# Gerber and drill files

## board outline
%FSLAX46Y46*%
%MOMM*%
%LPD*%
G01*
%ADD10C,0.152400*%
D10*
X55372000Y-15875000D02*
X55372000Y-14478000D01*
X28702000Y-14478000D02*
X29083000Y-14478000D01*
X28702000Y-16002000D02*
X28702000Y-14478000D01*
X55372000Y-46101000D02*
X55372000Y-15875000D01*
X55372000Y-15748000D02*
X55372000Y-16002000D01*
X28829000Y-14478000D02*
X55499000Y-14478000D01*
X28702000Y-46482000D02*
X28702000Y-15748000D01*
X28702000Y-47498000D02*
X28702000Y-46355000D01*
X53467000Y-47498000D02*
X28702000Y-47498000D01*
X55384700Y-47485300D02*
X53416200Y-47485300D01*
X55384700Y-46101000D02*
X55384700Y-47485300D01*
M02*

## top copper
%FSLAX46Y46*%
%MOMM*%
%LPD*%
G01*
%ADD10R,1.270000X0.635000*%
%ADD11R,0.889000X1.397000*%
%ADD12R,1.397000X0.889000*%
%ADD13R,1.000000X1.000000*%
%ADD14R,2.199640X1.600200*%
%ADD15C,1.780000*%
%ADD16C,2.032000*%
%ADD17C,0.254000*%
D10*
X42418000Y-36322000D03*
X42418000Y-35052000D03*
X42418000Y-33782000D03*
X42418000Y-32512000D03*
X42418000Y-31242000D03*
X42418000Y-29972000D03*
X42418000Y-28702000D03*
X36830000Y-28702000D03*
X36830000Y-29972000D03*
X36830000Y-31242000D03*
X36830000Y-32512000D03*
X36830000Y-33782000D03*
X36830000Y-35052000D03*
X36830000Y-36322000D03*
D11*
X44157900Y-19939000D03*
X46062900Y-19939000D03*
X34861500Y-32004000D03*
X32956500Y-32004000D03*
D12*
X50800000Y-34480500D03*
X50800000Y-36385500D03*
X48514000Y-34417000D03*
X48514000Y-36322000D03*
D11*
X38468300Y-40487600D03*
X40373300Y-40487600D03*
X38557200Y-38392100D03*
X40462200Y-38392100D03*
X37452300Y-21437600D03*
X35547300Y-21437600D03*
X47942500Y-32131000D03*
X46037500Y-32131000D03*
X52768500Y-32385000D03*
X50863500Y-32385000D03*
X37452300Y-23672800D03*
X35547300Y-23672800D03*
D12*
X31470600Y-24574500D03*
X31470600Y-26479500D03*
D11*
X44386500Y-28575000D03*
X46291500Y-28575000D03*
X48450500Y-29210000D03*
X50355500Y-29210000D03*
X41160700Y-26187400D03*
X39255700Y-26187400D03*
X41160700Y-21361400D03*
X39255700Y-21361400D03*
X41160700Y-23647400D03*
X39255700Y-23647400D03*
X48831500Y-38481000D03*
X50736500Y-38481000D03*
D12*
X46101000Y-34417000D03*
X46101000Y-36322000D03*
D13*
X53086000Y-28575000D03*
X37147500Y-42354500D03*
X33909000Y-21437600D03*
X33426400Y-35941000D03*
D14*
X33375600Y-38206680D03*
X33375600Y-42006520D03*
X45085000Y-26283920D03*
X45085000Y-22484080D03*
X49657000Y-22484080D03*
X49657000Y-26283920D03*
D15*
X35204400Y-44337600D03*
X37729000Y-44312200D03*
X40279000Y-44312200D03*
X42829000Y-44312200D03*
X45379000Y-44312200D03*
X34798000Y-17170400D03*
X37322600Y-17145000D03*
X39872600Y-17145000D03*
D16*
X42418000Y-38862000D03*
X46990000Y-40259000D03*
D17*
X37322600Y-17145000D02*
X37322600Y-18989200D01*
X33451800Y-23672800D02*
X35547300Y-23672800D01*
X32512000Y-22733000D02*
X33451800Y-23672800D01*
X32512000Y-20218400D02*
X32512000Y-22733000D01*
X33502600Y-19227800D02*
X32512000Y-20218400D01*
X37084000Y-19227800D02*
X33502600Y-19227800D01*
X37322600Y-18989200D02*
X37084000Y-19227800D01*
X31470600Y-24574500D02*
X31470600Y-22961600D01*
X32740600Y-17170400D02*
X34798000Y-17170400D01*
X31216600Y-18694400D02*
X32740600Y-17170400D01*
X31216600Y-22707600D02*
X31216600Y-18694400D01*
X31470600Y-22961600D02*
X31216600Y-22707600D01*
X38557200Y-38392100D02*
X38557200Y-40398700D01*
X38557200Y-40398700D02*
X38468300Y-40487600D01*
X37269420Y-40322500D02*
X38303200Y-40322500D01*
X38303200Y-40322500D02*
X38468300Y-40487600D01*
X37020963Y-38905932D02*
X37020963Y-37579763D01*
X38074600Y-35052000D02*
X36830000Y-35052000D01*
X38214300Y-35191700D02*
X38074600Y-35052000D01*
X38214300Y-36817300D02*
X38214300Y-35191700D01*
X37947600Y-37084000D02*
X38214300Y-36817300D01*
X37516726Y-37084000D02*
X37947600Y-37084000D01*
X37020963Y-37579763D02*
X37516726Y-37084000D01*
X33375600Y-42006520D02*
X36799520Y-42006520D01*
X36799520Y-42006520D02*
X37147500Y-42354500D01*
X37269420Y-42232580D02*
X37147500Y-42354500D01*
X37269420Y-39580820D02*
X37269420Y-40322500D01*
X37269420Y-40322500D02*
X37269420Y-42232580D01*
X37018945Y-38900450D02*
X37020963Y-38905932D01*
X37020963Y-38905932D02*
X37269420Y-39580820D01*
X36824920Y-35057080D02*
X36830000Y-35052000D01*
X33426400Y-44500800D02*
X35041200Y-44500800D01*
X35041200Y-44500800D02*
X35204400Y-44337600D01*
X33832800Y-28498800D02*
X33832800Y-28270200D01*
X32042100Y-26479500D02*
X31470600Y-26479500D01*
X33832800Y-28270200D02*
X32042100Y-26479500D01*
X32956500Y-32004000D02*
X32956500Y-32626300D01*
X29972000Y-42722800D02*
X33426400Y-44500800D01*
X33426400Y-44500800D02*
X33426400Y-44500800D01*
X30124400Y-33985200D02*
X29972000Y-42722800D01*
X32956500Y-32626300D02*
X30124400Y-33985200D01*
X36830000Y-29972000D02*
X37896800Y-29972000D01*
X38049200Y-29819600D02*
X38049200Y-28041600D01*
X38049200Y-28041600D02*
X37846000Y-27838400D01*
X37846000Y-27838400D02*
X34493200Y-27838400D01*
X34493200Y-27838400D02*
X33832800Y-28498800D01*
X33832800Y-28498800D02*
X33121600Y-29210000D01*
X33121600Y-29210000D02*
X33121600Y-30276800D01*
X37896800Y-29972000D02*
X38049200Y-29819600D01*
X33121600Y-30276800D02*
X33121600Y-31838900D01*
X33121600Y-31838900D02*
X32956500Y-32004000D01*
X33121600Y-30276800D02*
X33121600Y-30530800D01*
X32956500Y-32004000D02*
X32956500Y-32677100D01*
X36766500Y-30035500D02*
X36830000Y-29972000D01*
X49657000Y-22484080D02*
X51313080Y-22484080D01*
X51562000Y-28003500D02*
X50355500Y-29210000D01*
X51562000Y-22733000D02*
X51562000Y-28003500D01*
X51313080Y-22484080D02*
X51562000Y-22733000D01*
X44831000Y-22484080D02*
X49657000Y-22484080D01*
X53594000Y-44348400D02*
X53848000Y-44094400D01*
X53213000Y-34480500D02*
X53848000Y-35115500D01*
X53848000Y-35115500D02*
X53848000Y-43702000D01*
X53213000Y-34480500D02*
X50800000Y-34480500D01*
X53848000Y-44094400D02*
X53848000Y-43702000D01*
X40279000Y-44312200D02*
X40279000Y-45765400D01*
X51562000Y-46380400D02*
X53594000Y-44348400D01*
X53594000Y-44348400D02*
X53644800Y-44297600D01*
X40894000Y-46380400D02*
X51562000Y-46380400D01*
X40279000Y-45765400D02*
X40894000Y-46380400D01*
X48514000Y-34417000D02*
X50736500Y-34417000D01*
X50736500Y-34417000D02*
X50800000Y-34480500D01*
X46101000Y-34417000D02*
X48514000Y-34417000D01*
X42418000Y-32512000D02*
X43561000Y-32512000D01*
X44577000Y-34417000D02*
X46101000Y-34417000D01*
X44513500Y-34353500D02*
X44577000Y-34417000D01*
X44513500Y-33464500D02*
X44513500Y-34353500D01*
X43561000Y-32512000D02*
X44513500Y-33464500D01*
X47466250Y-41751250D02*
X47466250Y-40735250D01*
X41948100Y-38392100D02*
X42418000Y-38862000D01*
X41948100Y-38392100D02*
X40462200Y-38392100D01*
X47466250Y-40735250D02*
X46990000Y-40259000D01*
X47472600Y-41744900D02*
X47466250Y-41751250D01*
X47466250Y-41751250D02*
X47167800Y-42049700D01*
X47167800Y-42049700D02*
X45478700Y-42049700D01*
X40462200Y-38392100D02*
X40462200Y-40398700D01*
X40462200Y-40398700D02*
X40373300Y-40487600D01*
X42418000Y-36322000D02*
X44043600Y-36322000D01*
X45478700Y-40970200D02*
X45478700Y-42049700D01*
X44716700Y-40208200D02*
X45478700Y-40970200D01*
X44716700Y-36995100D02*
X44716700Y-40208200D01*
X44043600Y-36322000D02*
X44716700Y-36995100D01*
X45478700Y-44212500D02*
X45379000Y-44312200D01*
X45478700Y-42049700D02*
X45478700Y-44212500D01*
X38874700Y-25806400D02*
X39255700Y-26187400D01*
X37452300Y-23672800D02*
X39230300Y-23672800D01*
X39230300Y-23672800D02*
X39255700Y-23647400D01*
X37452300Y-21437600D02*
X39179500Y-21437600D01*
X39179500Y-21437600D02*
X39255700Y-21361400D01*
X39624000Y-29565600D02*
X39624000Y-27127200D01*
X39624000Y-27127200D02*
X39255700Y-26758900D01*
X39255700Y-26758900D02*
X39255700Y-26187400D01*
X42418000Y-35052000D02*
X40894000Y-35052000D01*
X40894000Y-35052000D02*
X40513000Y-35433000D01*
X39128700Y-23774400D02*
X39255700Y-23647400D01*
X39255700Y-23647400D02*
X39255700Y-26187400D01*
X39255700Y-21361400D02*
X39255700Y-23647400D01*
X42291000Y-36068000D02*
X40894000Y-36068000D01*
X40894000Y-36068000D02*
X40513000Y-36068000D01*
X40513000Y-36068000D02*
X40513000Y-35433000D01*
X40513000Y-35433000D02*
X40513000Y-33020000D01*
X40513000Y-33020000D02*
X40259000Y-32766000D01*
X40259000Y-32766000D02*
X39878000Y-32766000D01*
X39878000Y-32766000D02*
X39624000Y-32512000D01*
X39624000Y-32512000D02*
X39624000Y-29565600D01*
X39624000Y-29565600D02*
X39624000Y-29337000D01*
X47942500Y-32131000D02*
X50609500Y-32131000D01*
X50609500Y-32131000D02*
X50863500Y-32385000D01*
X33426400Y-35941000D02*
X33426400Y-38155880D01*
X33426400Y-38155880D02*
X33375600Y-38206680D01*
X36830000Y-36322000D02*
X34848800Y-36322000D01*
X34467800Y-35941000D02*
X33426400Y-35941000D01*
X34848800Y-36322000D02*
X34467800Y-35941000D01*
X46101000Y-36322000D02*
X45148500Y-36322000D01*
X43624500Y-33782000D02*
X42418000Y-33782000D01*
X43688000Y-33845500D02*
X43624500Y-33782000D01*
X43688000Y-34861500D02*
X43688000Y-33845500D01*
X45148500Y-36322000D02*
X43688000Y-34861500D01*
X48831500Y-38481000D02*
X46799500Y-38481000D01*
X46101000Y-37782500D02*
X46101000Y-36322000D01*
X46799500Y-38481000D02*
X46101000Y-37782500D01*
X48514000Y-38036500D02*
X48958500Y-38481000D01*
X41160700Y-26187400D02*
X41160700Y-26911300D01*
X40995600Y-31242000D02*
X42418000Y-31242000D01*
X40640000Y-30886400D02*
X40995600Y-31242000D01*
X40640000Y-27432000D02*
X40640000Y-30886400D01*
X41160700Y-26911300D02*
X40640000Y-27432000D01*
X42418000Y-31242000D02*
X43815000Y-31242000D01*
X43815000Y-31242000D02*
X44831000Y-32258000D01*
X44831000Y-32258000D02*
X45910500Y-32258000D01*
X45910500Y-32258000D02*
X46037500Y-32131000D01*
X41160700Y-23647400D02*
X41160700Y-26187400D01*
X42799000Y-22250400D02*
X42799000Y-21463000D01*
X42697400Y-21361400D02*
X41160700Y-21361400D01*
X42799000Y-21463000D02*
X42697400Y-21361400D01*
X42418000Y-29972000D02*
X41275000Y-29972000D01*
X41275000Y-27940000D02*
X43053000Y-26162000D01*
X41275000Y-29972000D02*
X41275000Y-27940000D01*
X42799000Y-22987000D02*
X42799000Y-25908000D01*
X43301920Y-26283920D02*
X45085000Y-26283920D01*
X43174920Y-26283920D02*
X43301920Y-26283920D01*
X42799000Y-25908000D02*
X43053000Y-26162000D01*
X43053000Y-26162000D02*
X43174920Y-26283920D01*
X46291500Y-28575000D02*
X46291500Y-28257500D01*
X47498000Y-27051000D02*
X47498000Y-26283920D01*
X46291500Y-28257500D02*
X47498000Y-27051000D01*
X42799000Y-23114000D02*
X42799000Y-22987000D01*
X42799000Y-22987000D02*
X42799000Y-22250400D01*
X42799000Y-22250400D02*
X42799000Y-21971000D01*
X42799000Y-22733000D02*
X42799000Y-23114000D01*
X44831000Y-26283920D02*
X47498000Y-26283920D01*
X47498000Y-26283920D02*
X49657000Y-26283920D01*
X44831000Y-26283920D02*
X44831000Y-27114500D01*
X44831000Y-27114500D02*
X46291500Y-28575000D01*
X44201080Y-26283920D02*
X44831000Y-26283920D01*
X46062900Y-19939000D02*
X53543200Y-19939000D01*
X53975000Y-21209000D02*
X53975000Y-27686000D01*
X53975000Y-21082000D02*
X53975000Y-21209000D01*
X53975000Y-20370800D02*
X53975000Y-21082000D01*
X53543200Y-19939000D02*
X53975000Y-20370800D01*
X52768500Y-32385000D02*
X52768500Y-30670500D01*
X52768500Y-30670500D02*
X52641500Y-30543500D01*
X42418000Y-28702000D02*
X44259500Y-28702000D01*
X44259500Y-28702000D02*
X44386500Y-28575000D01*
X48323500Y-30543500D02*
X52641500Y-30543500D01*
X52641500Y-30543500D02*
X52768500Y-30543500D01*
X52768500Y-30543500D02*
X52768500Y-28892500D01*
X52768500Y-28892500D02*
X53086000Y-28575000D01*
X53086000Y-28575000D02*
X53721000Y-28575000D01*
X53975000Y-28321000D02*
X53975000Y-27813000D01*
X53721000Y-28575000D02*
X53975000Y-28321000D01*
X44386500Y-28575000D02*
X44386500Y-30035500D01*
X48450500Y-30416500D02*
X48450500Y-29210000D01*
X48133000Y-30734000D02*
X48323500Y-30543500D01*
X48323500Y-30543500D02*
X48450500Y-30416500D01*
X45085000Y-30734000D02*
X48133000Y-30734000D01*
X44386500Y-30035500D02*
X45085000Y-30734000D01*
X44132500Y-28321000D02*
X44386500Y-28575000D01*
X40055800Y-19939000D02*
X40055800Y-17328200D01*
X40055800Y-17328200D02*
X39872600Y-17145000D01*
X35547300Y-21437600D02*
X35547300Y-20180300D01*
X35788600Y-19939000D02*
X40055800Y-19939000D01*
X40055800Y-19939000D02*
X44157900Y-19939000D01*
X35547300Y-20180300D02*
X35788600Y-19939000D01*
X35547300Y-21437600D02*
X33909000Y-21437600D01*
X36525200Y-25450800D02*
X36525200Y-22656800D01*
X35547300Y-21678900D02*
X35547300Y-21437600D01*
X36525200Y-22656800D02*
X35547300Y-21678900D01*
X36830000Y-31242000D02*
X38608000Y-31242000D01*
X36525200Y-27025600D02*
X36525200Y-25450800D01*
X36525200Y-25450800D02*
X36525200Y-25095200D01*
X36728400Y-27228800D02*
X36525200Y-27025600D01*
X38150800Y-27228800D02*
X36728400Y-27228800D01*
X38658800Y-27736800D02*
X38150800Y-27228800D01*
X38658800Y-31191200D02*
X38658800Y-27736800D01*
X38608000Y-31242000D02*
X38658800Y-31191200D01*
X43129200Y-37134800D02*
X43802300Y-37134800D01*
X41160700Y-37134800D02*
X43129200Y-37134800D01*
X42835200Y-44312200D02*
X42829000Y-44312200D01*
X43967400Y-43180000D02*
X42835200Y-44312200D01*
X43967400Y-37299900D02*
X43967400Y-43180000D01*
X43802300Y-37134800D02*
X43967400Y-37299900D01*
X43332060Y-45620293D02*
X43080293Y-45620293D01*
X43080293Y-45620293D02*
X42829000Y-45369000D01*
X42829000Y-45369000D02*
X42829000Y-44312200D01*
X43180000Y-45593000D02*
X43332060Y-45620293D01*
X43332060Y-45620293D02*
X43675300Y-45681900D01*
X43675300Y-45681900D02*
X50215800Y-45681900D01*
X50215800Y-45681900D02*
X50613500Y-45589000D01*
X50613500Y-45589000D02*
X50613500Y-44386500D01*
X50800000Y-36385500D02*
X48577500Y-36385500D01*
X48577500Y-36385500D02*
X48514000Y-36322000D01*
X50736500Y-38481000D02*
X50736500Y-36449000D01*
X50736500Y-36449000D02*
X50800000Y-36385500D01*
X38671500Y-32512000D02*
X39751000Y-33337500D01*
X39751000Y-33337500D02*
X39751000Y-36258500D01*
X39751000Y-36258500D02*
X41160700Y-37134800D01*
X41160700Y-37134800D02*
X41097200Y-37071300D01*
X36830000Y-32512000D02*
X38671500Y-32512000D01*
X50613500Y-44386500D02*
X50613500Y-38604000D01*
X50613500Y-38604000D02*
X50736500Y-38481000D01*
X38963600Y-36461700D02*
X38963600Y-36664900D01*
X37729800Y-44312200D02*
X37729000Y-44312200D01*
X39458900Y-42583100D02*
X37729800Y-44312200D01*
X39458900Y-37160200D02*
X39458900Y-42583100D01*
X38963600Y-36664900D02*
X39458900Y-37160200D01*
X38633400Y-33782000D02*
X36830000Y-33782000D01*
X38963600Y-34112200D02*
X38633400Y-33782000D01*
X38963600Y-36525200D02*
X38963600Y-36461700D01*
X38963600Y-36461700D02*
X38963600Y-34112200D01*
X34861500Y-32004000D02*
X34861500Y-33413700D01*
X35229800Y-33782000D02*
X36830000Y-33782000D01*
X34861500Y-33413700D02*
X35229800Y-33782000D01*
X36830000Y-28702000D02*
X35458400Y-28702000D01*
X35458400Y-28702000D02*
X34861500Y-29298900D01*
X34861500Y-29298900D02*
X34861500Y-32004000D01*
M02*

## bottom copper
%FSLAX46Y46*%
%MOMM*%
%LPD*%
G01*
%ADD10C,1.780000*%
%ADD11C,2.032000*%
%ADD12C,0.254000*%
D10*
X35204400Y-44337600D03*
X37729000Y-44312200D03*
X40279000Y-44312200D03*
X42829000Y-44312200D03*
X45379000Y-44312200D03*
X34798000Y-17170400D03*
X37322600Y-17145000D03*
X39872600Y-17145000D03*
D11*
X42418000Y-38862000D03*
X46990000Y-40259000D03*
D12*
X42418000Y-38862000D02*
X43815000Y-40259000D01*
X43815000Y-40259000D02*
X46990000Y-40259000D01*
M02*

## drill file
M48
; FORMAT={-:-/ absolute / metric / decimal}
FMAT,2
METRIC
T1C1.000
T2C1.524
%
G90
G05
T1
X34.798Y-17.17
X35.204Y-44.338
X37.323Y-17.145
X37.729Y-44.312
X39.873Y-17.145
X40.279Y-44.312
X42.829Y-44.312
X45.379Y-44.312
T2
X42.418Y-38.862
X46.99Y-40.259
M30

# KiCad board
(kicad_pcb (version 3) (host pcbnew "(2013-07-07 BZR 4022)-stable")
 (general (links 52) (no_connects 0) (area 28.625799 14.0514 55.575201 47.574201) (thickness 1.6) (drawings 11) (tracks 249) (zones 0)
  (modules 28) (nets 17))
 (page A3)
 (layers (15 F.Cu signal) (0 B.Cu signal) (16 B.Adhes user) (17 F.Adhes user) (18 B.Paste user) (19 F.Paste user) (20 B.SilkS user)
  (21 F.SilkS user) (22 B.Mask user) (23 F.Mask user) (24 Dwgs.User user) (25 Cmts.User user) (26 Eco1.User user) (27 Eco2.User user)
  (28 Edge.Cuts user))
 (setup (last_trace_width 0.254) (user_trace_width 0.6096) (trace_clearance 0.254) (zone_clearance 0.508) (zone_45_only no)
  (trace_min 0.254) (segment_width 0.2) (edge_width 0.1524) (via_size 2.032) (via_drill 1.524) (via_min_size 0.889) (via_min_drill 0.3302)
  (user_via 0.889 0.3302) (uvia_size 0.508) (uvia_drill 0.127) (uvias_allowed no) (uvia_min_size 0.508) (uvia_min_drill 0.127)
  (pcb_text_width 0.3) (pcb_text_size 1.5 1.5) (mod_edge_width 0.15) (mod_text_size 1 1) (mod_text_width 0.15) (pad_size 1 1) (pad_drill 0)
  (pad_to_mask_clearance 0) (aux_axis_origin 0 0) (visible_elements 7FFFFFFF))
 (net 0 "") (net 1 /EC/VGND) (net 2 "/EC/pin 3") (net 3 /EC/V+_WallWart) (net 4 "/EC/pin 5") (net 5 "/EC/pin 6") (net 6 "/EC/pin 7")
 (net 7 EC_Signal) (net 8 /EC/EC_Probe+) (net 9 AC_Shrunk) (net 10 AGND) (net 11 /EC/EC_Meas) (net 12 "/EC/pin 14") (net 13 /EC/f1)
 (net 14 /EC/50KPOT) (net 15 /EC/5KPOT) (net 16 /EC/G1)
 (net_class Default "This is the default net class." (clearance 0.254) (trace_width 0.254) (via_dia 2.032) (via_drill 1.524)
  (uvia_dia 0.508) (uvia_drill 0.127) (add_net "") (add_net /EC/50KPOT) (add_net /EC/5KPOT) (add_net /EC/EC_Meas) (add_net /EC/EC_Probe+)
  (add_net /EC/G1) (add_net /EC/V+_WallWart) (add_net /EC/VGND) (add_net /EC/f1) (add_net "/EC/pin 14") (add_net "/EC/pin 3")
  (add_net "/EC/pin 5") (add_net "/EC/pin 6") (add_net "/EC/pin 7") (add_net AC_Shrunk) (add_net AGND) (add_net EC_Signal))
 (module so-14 (layer F.Cu) (at 39.624 32.512 90)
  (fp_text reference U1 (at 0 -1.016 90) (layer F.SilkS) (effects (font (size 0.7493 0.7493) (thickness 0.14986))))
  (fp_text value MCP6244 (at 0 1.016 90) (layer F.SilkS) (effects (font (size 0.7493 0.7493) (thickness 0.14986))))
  (pad 1 smd rect (at -3.81 2.794 90) (size 0.635 1.27) (layers F.Cu F.Paste F.Mask) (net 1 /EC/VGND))
  (pad 2 smd rect (at -2.54 2.794 90) (size 0.635 1.27) (layers F.Cu F.Paste F.Mask) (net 1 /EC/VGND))
  (pad 3 smd rect (at -1.27 2.794 90) (size 0.635 1.27) (layers F.Cu F.Paste F.Mask) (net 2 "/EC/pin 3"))
  (pad 4 smd rect (at 0 2.794 90) (size 0.635 1.27) (layers F.Cu F.Paste F.Mask) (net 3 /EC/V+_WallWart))
  (pad 5 smd rect (at 1.27 2.794 90) (size 0.635 1.27) (layers F.Cu F.Paste F.Mask) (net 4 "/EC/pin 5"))
  (pad 6 smd rect (at 2.54 2.794 90) (size 0.635 1.27) (layers F.Cu F.Paste F.Mask) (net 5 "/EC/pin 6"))
  (pad 7 smd rect (at 3.81 2.794 90) (size 0.635 1.27) (layers F.Cu F.Paste F.Mask) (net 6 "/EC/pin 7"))
  (pad 8 smd rect (at 3.81 -2.794 90) (size 0.635 1.27) (layers F.Cu F.Paste F.Mask) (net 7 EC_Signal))
  (pad 9 smd rect (at 2.54 -2.794 90) (size 0.635 1.27) (layers F.Cu F.Paste F.Mask) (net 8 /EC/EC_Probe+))
  (pad 10 smd rect (at 1.27 -2.794 90) (size 0.635 1.27) (layers F.Cu F.Paste F.Mask) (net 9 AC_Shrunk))
  (pad 11 smd rect (at 0 -2.794 90) (size 0.635 1.27) (layers F.Cu F.Paste F.Mask) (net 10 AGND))
  (pad 12 smd rect (at -1.27 -2.794 90) (size 0.635 1.27) (layers F.Cu F.Paste F.Mask) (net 7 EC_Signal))
  (pad 13 smd rect (at -2.54 -2.794 90) (size 0.635 1.27) (layers F.Cu F.Paste F.Mask) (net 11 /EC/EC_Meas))
  (pad 14 smd rect (at -3.81 -2.794 90) (size 0.635 1.27) (layers F.Cu F.Paste F.Mask) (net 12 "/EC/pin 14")))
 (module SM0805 (layer F.Cu) (at 45.1104 19.939)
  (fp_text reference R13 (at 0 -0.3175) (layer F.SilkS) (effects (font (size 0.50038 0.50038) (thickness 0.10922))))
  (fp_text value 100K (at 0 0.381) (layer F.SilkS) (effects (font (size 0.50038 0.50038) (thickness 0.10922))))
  (pad 1 smd rect (at -0.9525 0) (size 0.889 1.397) (layers F.Cu F.Paste F.Mask) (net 9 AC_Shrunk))
  (pad 2 smd rect (at 0.9525 0) (size 0.889 1.397) (layers F.Cu F.Paste F.Mask) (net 6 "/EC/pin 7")))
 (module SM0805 (layer F.Cu) (at 33.909 32.004 180)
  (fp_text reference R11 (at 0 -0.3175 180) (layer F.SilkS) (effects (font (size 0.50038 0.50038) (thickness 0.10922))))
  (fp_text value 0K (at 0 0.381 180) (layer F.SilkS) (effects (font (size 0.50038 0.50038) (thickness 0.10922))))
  (pad 1 smd rect (at -0.9525 0 180) (size 0.889 1.397) (layers F.Cu F.Paste F.Mask) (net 7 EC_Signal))
  (pad 2 smd rect (at 0.9525 0 180) (size 0.889 1.397) (layers F.Cu F.Paste F.Mask) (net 8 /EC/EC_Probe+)))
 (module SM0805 (layer F.Cu) (at 50.8 35.433 270)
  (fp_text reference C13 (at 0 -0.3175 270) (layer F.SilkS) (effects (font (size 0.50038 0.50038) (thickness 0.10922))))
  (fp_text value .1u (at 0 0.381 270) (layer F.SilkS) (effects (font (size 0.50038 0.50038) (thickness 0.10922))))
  (pad 1 smd rect (at -0.9525 0 270) (size 0.889 1.397) (layers F.Cu F.Paste F.Mask) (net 3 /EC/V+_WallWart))
  (pad 2 smd rect (at 0.9525 0 270) (size 0.889 1.397) (layers F.Cu F.Paste F.Mask) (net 10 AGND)))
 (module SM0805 (layer F.Cu) (at 48.514 35.3695 270)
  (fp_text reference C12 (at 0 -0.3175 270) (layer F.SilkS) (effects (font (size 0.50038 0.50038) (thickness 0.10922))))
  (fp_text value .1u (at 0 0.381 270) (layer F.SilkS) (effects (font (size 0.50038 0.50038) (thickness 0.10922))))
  (pad 1 smd rect (at -0.9525 0 270) (size 0.889 1.397) (layers F.Cu F.Paste F.Mask) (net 3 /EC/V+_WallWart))
  (pad 2 smd rect (at 0.9525 0 270) (size 0.889 1.397) (layers F.Cu F.Paste F.Mask) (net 10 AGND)))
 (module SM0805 (layer F.Cu) (at 39.4208 40.4876)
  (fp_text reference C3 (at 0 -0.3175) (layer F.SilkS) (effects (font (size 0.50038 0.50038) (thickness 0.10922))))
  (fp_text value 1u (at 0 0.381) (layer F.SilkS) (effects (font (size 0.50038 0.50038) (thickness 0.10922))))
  (pad 1 smd rect (at -0.9525 0) (size 0.889 1.397) (layers F.Cu F.Paste F.Mask) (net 11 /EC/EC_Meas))
  (pad 2 smd rect (at 0.9525 0) (size 0.889 1.397) (layers F.Cu F.Paste F.Mask) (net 1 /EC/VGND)))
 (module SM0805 (layer F.Cu) (at 39.5097 38.3921)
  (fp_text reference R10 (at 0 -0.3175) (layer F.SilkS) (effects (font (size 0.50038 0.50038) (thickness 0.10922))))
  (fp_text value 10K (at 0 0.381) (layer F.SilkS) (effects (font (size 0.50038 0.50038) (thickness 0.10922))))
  (pad 1 smd rect (at -0.9525 0) (size 0.889 1.397) (layers F.Cu F.Paste F.Mask) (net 11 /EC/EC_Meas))
  (pad 2 smd rect (at 0.9525 0) (size 0.889 1.397) (layers F.Cu F.Paste F.Mask) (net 1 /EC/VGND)))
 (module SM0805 (layer F.Cu) (at 36.4998 21.4376 180)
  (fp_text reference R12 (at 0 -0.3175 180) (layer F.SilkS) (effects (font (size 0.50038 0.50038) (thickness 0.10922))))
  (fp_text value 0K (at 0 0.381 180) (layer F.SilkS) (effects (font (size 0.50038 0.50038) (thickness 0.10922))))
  (pad 1 smd rect (at -0.9525 0 180) (size 0.889 1.397) (layers F.Cu F.Paste F.Mask) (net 1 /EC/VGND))
  (pad 2 smd rect (at 0.9525 0 180) (size 0.889 1.397) (layers F.Cu F.Paste F.Mask) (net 9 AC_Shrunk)))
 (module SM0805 (layer F.Cu) (at 46.99 32.131 180)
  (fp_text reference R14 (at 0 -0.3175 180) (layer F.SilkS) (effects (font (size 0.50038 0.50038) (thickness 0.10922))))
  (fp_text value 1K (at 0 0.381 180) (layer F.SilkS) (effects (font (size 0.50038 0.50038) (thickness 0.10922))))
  (pad 1 smd rect (at -0.9525 0 180) (size 0.889 1.397) (layers F.Cu F.Paste F.Mask) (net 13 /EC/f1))
  (pad 2 smd rect (at 0.9525 0 180) (size 0.889 1.397) (layers F.Cu F.Paste F.Mask) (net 4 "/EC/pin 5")))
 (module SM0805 (layer F.Cu) (at 51.816 32.385 180)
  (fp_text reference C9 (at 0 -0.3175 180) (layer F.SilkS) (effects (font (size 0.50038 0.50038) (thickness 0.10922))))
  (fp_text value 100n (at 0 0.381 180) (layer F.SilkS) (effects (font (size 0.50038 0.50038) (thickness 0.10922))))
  (pad 1 smd rect (at -0.9525 0 180) (size 0.889 1.397) (layers F.Cu F.Paste F.Mask) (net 6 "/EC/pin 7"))
  (pad 2 smd rect (at 0.9525 0 180) (size 0.889 1.397) (layers F.Cu F.Paste F.Mask) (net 13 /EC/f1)))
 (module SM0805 (layer F.Cu) (at 36.4998 23.6728 180)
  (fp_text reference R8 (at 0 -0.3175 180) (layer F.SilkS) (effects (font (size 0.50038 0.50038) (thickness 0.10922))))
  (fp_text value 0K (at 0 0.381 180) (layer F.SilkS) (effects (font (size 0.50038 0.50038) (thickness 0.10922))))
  (pad 1 smd rect (at -0.9525 0 180) (size 0.889 1.397) (layers F.Cu F.Paste F.Mask) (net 1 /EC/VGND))
  (pad 2 smd rect (at 0.9525 0 180) (size 0.889 1.397) (layers F.Cu F.Paste F.Mask) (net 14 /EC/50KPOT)))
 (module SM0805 (layer F.Cu) (at 31.4706 25.527 270)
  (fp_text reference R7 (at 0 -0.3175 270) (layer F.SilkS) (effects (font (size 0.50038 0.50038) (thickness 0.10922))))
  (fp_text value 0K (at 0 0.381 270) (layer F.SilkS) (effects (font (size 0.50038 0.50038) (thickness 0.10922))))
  (pad 1 smd rect (at -0.9525 0 270) (size 0.889 1.397) (layers F.Cu F.Paste F.Mask) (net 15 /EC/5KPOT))
  (pad 2 smd rect (at 0.9525 0 270) (size 0.889 1.397) (layers F.Cu F.Paste F.Mask) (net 8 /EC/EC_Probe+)))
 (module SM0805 (layer F.Cu) (at 45.339 28.575)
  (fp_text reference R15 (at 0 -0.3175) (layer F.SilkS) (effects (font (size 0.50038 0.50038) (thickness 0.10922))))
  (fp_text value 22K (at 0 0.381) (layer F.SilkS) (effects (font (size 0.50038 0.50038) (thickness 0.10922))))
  (pad 1 smd rect (at -0.9525 0) (size 0.889 1.397) (layers F.Cu F.Paste F.Mask) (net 6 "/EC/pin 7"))
  (pad 2 smd rect (at 0.9525 0) (size 0.889 1.397) (layers F.Cu F.Paste F.Mask) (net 5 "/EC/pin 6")))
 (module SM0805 (layer F.Cu) (at 49.403 29.21)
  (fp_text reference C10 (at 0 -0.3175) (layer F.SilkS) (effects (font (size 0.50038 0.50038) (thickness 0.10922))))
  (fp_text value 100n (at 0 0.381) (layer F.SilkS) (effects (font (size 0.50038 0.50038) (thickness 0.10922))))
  (pad 1 smd rect (at -0.9525 0) (size 0.889 1.397) (layers F.Cu F.Paste F.Mask) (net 6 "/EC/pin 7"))
  (pad 2 smd rect (at 0.9525 0) (size 0.889 1.397) (layers F.Cu F.Paste F.Mask) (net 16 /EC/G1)))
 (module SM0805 (layer F.Cu) (at 40.2082 26.1874 180)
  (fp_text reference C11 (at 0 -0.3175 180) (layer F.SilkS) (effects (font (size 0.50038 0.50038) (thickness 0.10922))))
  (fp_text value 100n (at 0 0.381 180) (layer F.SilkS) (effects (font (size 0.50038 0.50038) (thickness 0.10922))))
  (pad 1 smd rect (at -0.9525 0 180) (size 0.889 1.397) (layers F.Cu F.Paste F.Mask) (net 4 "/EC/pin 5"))
  (pad 2 smd rect (at 0.9525 0 180) (size 0.889 1.397) (layers F.Cu F.Paste F.Mask) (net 1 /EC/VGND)))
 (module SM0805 (layer F.Cu) (at 40.2082 21.3614 180)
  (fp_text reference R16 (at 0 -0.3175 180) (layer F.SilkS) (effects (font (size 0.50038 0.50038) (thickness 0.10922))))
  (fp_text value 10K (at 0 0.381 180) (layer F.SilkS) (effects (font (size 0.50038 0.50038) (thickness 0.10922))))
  (pad 1 smd rect (at -0.9525 0 180) (size 0.889 1.397) (layers F.Cu F.Paste F.Mask) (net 5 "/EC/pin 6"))
  (pad 2 smd rect (at 0.9525 0 180) (size 0.889 1.397) (layers F.Cu F.Paste F.Mask) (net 1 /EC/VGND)))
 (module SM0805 (layer F.Cu) (at 40.2082 23.6474 180)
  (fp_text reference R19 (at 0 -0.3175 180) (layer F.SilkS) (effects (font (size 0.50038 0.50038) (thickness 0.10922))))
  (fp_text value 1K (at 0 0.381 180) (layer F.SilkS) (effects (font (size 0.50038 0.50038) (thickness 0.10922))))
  (pad 1 smd rect (at -0.9525 0 180) (size 0.889 1.397) (layers F.Cu F.Paste F.Mask) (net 4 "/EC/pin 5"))
  (pad 2 smd rect (at 0.9525 0 180) (size 0.889 1.397) (layers F.Cu F.Paste F.Mask) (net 1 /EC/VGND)))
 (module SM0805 (layer F.Cu) (at 49.784 38.481)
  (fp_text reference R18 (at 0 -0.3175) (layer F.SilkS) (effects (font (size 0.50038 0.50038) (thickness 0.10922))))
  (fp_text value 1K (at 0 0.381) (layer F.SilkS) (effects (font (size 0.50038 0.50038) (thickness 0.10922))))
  (pad 1 smd rect (at -0.9525 0) (size 0.889 1.397) (layers F.Cu F.Paste F.Mask) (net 2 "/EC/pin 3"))
  (pad 2 smd rect (at 0.9525 0) (size 0.889 1.397) (layers F.Cu F.Paste F.Mask) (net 10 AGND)))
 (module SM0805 (layer F.Cu) (at 46.101 35.3695 270)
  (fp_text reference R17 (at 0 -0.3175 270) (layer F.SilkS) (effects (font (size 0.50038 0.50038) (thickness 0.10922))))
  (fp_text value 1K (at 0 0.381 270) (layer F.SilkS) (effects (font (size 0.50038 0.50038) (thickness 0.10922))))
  (pad 1 smd rect (at -0.9525 0 270) (size 0.889 1.397) (layers F.Cu F.Paste F.Mask) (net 3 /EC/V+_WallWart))
  (pad 2 smd rect (at 0.9525 0 270) (size 0.889 1.397) (layers F.Cu F.Paste F.Mask) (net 2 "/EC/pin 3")))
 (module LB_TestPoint (layer F.Cu) (at 53.086 28.575)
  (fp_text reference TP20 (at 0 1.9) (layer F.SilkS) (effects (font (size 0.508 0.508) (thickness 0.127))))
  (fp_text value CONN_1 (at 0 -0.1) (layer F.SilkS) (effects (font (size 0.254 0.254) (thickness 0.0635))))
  (pad 1 smd rect (at 0 0) (size 1 1) (layers F.Cu F.Paste F.Mask) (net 6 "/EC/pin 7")))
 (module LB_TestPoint (layer F.Cu) (at 37.1475 42.3545 90)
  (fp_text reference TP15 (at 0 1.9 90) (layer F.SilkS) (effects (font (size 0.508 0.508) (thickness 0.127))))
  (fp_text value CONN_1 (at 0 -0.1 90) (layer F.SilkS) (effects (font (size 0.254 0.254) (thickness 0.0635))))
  (pad 1 smd rect (at 0 0 90) (size 1 1) (layers F.Cu F.Paste F.Mask) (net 11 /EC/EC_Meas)))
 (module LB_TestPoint (layer F.Cu) (at 33.909 21.4376)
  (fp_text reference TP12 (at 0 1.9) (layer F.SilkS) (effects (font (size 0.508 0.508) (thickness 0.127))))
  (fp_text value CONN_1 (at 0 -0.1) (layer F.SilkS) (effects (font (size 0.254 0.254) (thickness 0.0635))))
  (pad 1 smd rect (at 0 0) (size 1 1) (layers F.Cu F.Paste F.Mask) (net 9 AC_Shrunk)))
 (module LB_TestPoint (layer F.Cu) (at 33.4264 35.941)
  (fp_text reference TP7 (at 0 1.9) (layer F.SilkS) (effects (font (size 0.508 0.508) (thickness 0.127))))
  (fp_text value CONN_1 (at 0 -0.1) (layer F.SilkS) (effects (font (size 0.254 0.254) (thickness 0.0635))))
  (pad 1 smd rect (at 0 0) (size 1 1) (layers F.Cu F.Paste F.Mask) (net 12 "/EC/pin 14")))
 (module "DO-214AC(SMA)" (layer F.Cu) (at 33.3756 40.1066 270)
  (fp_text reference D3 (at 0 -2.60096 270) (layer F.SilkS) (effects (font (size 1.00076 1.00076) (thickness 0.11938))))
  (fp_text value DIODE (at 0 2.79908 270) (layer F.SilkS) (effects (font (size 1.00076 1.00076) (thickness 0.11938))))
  (pad 1 smd rect (at -1.89992 0 270) (size 1.6002 2.19964) (layers F.Cu F.Paste F.Mask) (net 12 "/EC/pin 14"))
  (pad 2 smd rect (at 1.89992 0 270) (size 1.6002 2.19964) (layers F.Cu F.Paste F.Mask) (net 11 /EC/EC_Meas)))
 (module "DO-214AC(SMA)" (layer F.Cu) (at 45.085 24.384 90)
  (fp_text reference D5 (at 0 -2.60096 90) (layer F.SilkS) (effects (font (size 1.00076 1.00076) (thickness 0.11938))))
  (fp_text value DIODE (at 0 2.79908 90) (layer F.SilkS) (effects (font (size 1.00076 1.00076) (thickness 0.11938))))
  (pad 1 smd rect (at -1.89992 0 90) (size 1.6002 2.19964) (layers F.Cu F.Paste F.Mask) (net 5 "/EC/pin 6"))
  (pad 2 smd rect (at 1.89992 0 90) (size 1.6002 2.19964) (layers F.Cu F.Paste F.Mask) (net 16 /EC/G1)))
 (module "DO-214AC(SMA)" (layer F.Cu) (at 49.657 24.384 270)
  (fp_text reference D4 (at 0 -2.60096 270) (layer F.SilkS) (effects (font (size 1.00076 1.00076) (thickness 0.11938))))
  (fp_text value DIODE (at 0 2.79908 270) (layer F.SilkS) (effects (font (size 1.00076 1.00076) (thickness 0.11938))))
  (pad 1 smd rect (at -1.89992 0 270) (size 1.6002 2.19964) (layers F.Cu F.Paste F.Mask) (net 16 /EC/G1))
  (pad 2 smd rect (at 1.89992 0 270) (size 1.6002 2.19964) (layers F.Cu F.Paste F.Mask) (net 5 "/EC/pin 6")))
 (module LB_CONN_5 (layer F.Cu) (at 35.2044 44.2976)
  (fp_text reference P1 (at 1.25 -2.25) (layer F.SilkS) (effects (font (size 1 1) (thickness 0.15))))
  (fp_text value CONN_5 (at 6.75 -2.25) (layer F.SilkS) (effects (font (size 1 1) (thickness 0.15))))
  (pad 1 thru_hole circle (at 0 0.04) (size 1.78 1.78) (drill 1) (layers *.Cu *.Mask F.SilkS) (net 8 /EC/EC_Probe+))
  (pad 2 thru_hole circle (at 2.5246 0.0146) (size 1.78 1.78) (drill 1) (layers *.Cu *.Mask F.SilkS) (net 7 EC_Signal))
  (pad 3 thru_hole circle (at 5.0746 0.0146) (size 1.78 1.78) (drill 1) (layers *.Cu *.Mask F.SilkS) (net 3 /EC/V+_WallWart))
  (pad 4 thru_hole circle (at 7.6246 0.0146) (size 1.78 1.78) (drill 1) (layers *.Cu *.Mask F.SilkS) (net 10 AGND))
  (pad 5 thru_hole circle (at 10.1746 0.0146) (size 1.78 1.78) (drill 1) (layers *.Cu *.Mask F.SilkS) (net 1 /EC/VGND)))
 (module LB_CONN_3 (layer F.Cu) (at 34.798 14.6304)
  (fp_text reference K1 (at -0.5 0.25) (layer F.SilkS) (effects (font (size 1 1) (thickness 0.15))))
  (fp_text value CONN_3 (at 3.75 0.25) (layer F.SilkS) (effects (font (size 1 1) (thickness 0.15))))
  (pad 1 thru_hole circle (at 0 2.54) (size 1.78 1.78) (drill 1) (layers *.Cu *.Mask F.SilkS) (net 15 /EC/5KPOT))
  (pad 2 thru_hole circle (at 2.5246 2.5146) (size 1.78 1.78) (drill 1) (layers *.Cu *.Mask F.SilkS) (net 14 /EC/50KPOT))
  (pad 3 thru_hole circle (at 5.0746 2.5146) (size 1.78 1.78) (drill 1) (layers *.Cu *.Mask F.SilkS) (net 9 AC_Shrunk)))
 (gr_line (start 55.372 15.875) (end 55.372 14.478) (angle 90) (layer Edge.Cuts) (width 0.1524))
 (gr_line (start 28.702 14.478) (end 29.083 14.478) (angle 90) (layer Edge.Cuts) (width 0.1524))
 (gr_line (start 28.702 16.002) (end 28.702 14.478) (angle 90) (layer Edge.Cuts) (width 0.1524))
 (gr_line (start 55.372 46.101) (end 55.372 15.875) (angle 90) (layer Edge.Cuts) (width 0.1524))
 (gr_line (start 55.372 15.748) (end 55.372 16.002) (angle 90) (layer Edge.Cuts) (width 0.1524))
 (gr_line (start 28.829 14.478) (end 55.499 14.478) (angle 90) (layer Edge.Cuts) (width 0.1524))
 (gr_line (start 28.702 46.482) (end 28.702 15.748) (angle 90) (layer Edge.Cuts) (width 0.1524))
 (gr_line (start 28.702 47.498) (end 28.702 46.355) (angle 90) (layer Edge.Cuts) (width 0.1524))
 (gr_line (start 53.467 47.498) (end 28.702 47.498) (angle 90) (layer Edge.Cuts) (width 0.1524))
 (gr_line (start 55.3847 47.4853) (end 53.4162 47.4853) (angle 90) (layer Edge.Cuts) (width 0.1524))
 (gr_line (start 55.3847 46.101) (end 55.3847 47.4853) (angle 90) (layer Edge.Cuts) (width 0.1524))
 (segment (start 37.3226 17.145) (end 37.3226 18.9892) (width 0.254) (layer F.Cu) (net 14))
 (segment (start 33.4518 23.6728) (end 35.5473 23.6728) (width 0.254) (layer F.Cu) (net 14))
 (segment (start 32.512 22.733) (end 33.4518 23.6728) (width 0.254) (layer F.Cu) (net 14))
 (segment (start 32.512 20.2184) (end 32.512 22.733) (width 0.254) (layer F.Cu) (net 14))
 (segment (start 33.5026 19.2278) (end 32.512 20.2184) (width 0.254) (layer F.Cu) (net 14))
 (segment (start 37.084 19.2278) (end 33.5026 19.2278) (width 0.254) (layer F.Cu) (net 14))
 (segment (start 37.3226 18.9892) (end 37.084 19.2278) (width 0.254) (layer F.Cu) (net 14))
 (segment (start 31.4706 24.5745) (end 31.4706 22.9616) (width 0.254) (layer F.Cu) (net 15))
 (segment (start 32.7406 17.1704) (end 34.798 17.1704) (width 0.254) (layer F.Cu) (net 15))
 (segment (start 31.2166 18.6944) (end 32.7406 17.1704) (width 0.254) (layer F.Cu) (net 15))
 (segment (start 31.2166 22.7076) (end 31.2166 18.6944) (width 0.254) (layer F.Cu) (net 15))
 (segment (start 31.4706 22.9616) (end 31.2166 22.7076) (width 0.254) (layer F.Cu) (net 15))
 (segment (start 38.5572 38.3921) (end 38.5572 40.3987) (width 0.254) (layer F.Cu) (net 11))
 (segment (start 38.5572 40.3987) (end 38.4683 40.4876) (width 0.254) (layer F.Cu) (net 11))
 (segment (start 37.26942 40.3225) (end 38.3032 40.3225) (width 0.254) (layer F.Cu) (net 11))
 (segment (start 38.3032 40.3225) (end 38.4683 40.4876) (width 0.254) (layer F.Cu) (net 11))
 (segment (start 37.020963 38.905932) (end 37.020963 37.579763) (width 0.254) (layer F.Cu) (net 11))
 (segment (start 38.0746 35.052) (end 36.83 35.052) (width 0.254) (layer F.Cu) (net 11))
 (segment (start 38.2143 35.1917) (end 38.0746 35.052) (width 0.254) (layer F.Cu) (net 11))
 (segment (start 38.2143 36.8173) (end 38.2143 35.1917) (width 0.254) (layer F.Cu) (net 11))
 (segment (start 37.9476 37.084) (end 38.2143 36.8173) (width 0.254) (layer F.Cu) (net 11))
 (segment (start 37.516726 37.084) (end 37.9476 37.084) (width 0.254) (layer F.Cu) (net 11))
 (segment (start 37.020963 37.579763) (end 37.516726 37.084) (width 0.254) (layer F.Cu) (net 11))
 (segment (start 33.3756 42.00652) (end 36.79952 42.00652) (width 0.254) (layer F.Cu) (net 11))
 (segment (start 36.79952 42.00652) (end 37.1475 42.3545) (width 0.254) (layer F.Cu) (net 11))
 (segment (start 37.26942 42.23258) (end 37.1475 42.3545) (width 0.254) (layer F.Cu) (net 11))
 (segment (start 37.26942 39.58082) (end 37.26942 40.3225) (width 0.254) (layer F.Cu) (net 11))
 (segment (start 37.26942 40.3225) (end 37.26942 42.23258) (width 0.254) (layer F.Cu) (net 11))
 (segment (start 37.018945 38.90045) (end 37.020963 38.905932) (width 0.254) (layer F.Cu) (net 11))
 (segment (start 37.020963 38.905932) (end 37.26942 39.58082) (width 0.254) (layer F.Cu) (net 11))
 (segment (start 36.82492 35.05708) (end 36.83 35.052) (width 0.254) (layer F.Cu) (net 11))
 (segment (start 33.4264 44.5008) (end 35.0412 44.5008) (width 0.254) (layer F.Cu) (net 8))
 (segment (start 35.0412 44.5008) (end 35.2044 44.3376) (width 0.254) (layer F.Cu) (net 8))
 (segment (start 33.8328 28.4988) (end 33.8328 28.2702) (width 0.254) (layer F.Cu) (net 8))
 (segment (start 32.0421 26.4795) (end 31.4706 26.4795) (width 0.254) (layer F.Cu) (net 8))
 (segment (start 33.8328 28.2702) (end 32.0421 26.4795) (width 0.254) (layer F.Cu) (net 8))
 (segment (start 32.9565 32.004) (end 32.9565 32.6263) (width 0.254) (layer F.Cu) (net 8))
 (segment (start 29.972 42.7228) (end 33.4264 44.5008) (width 0.254) (layer F.Cu) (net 8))
 (segment (start 33.4264 44.5008) (end 33.4264 44.5008) (width 0.254) (layer F.Cu) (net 8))
 (segment (start 30.1244 33.9852) (end 29.972 42.7228) (width 0.254) (layer F.Cu) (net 8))
 (segment (start 32.9565 32.6263) (end 30.1244 33.9852) (width 0.254) (layer F.Cu) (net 8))
 (segment (start 36.83 29.972) (end 37.8968 29.972) (width 0.254) (layer F.Cu) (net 8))
 (segment (start 38.0492 29.8196) (end 38.0492 28.0416) (width 0.254) (layer F.Cu) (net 8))
 (segment (start 38.0492 28.0416) (end 37.846 27.8384) (width 0.254) (layer F.Cu) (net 8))
 (segment (start 37.846 27.8384) (end 34.4932 27.8384) (width 0.254) (layer F.Cu) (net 8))
 (segment (start 34.4932 27.8384) (end 33.8328 28.4988) (width 0.254) (layer F.Cu) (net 8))
 (segment (start 33.8328 28.4988) (end 33.1216 29.21) (width 0.254) (layer F.Cu) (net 8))
 (segment (start 33.1216 29.21) (end 33.1216 30.2768) (width 0.254) (layer F.Cu) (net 8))
 (segment (start 37.8968 29.972) (end 38.0492 29.8196) (width 0.254) (layer F.Cu) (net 8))
 (segment (start 33.1216 30.2768) (end 33.1216 31.8389) (width 0.254) (layer F.Cu) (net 8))
 (segment (start 33.1216 31.8389) (end 32.9565 32.004) (width 0.254) (layer F.Cu) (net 8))
 (segment (start 33.1216 30.2768) (end 33.1216 30.5308) (width 0.254) (layer F.Cu) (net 8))
 (segment (start 32.9565 32.004) (end 32.9565 32.6771) (width 0.254) (layer F.Cu) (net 8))
 (segment (start 36.7665 30.0355) (end 36.83 29.972) (width 0.254) (layer F.Cu) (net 8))
 (segment (start 49.657 22.48408) (end 51.31308 22.48408) (width 0.254) (layer F.Cu) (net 16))
 (segment (start 51.562 28.0035) (end 50.3555 29.21) (width 0.254) (layer F.Cu) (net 16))
 (segment (start 51.562 22.733) (end 51.562 28.0035) (width 0.254) (layer F.Cu) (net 16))
 (segment (start 51.31308 22.48408) (end 51.562 22.733) (width 0.254) (layer F.Cu) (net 16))
 (segment (start 44.831 22.48408) (end 49.657 22.48408) (width 0.254) (layer F.Cu) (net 16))
 (segment (start 53.594 44.3484) (end 53.848 44.0944) (width 0.254) (layer F.Cu) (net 3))
 (segment (start 53.213 34.4805) (end 53.848 35.1155) (width 0.254) (layer F.Cu) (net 3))
 (segment (start 53.848 35.1155) (end 53.848 43.702) (width 0.254) (layer F.Cu) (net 3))
 (segment (start 53.213 34.4805) (end 50.8 34.4805) (width 0.254) (layer F.Cu) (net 3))
 (segment (start 53.848 44.0944) (end 53.848 43.702) (width 0.254) (layer F.Cu) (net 3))
 (segment (start 40.279 44.3122) (end 40.279 45.7654) (width 0.254) (layer F.Cu) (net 3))
 (segment (start 51.562 46.3804) (end 53.594 44.3484) (width 0.254) (layer F.Cu) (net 3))
 (segment (start 53.594 44.3484) (end 53.6448 44.2976) (width 0.254) (layer F.Cu) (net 3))
 (segment (start 40.894 46.3804) (end 51.562 46.3804) (width 0.254) (layer F.Cu) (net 3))
 (segment (start 40.279 45.7654) (end 40.894 46.3804) (width 0.254) (layer F.Cu) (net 3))
 (segment (start 48.514 34.417) (end 50.7365 34.417) (width 0.254) (layer F.Cu) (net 3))
 (segment (start 50.7365 34.417) (end 50.8 34.4805) (width 0.254) (layer F.Cu) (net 3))
 (segment (start 46.101 34.417) (end 48.514 34.417) (width 0.254) (layer F.Cu) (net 3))
 (segment (start 42.418 32.512) (end 43.561 32.512) (width 0.254) (layer F.Cu) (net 3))
 (segment (start 44.577 34.417) (end 46.101 34.417) (width 0.254) (layer F.Cu) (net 3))
 (segment (start 44.5135 34.3535) (end 44.577 34.417) (width 0.254) (layer F.Cu) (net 3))
 (segment (start 44.5135 33.4645) (end 44.5135 34.3535) (width 0.254) (layer F.Cu) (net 3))
 (segment (start 43.561 32.512) (end 44.5135 33.4645) (width 0.254) (layer F.Cu) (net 3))
 (segment (start 47.46625 41.75125) (end 47.46625 40.73525) (width 0.254) (layer F.Cu) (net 1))
 (segment (start 41.9481 38.3921) (end 42.418 38.862) (width 0.254) (layer F.Cu) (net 1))
 (via (at 42.418 38.862) (size 2.032) (layers F.Cu B.Cu) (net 1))
 (segment (start 42.418 38.862) (end 43.815 40.259) (width 0.254) (layer B.Cu) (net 1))
 (segment (start 43.815 40.259) (end 46.99 40.259) (width 0.254) (layer B.Cu) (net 1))
 (via (at 46.99 40.259) (size 2.032) (layers F.Cu B.Cu) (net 1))
 (segment (start 41.9481 38.3921) (end 40.4622 38.3921) (width 0.254) (layer F.Cu) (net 1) (status 800000))
 (segment (start 47.46625 40.73525) (end 46.99 40.259) (width 0.254) (layer F.Cu) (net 1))
 (segment (start 47.4726 41.7449) (end 47.46625 41.75125) (width 0.254) (layer F.Cu) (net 1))
 (segment (start 47.46625 41.75125) (end 47.1678 42.0497) (width 0.254) (layer F.Cu) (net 1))
 (segment (start 47.1678 42.0497) (end 45.4787 42.0497) (width 0.254) (layer F.Cu) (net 1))
 (segment (start 40.4622 38.3921) (end 40.4622 40.3987) (width 0.254) (layer F.Cu) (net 1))
 (segment (start 40.4622 40.3987) (end 40.3733 40.4876) (width 0.254) (layer F.Cu) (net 1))
 (segment (start 42.418 36.322) (end 44.0436 36.322) (width 0.254) (layer F.Cu) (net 1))
 (segment (start 45.4787 40.9702) (end 45.4787 42.0497) (width 0.254) (layer F.Cu) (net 1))
 (segment (start 44.7167 40.2082) (end 45.4787 40.9702) (width 0.254) (layer F.Cu) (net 1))
 (segment (start 44.7167 36.9951) (end 44.7167 40.2082) (width 0.254) (layer F.Cu) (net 1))
 (segment (start 44.0436 36.322) (end 44.7167 36.9951) (width 0.254) (layer F.Cu) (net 1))
 (segment (start 45.4787 44.2125) (end 45.379 44.3122) (width 0.254) (layer F.Cu) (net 1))
 (segment (start 45.4787 42.0497) (end 45.4787 44.2125) (width 0.254) (layer F.Cu) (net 1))
 (segment (start 38.8747 25.8064) (end 39.2557 26.1874) (width 0.254) (layer F.Cu) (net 1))
 (segment (start 37.4523 23.6728) (end 39.2303 23.6728) (width 0.254) (layer F.Cu) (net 1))
 (segment (start 39.2303 23.6728) (end 39.2557 23.6474) (width 0.254) (layer F.Cu) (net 1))
 (segment (start 37.4523 21.4376) (end 39.1795 21.4376) (width 0.254) (layer F.Cu) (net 1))
 (segment (start 39.1795 21.4376) (end 39.2557 21.3614) (width 0.254) (layer F.Cu) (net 1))
 (segment (start 39.624 29.5656) (end 39.624 27.1272) (width 0.254) (layer F.Cu) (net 1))
 (segment (start 39.624 27.1272) (end 39.2557 26.7589) (width 0.254) (layer F.Cu) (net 1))
 (segment (start 39.2557 26.7589) (end 39.2557 26.1874) (width 0.254) (layer F.Cu) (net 1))
 (segment (start 42.418 35.052) (end 40.894 35.052) (width 0.254) (layer F.Cu) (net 1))
 (segment (start 40.894 35.052) (end 40.513 35.433) (width 0.254) (layer F.Cu) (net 1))
 (segment (start 39.1287 23.7744) (end 39.2557 23.6474) (width 0.254) (layer F.Cu) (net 1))
 (segment (start 39.2557 23.6474) (end 39.2557 26.1874) (width 0.254) (layer F.Cu) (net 1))
 (segment (start 39.2557 21.3614) (end 39.2557 23.6474) (width 0.254) (layer F.Cu) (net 1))
 (segment (start 42.291 36.068) (end 40.894 36.068) (width 0.254) (layer F.Cu) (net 1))
 (segment (start 40.894 36.068) (end 40.513 36.068) (width 0.254) (layer F.Cu) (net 1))
 (segment (start 40.513 36.068) (end 40.513 35.433) (width 0.254) (layer F.Cu) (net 1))
 (segment (start 40.513 35.433) (end 40.513 33.02) (width 0.254) (layer F.Cu) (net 1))
 (segment (start 40.513 33.02) (end 40.259 32.766) (width 0.254) (layer F.Cu) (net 1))
 (segment (start 40.259 32.766) (end 39.878 32.766) (width 0.254) (layer F.Cu) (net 1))
 (segment (start 39.878 32.766) (end 39.624 32.512) (width 0.254) (layer F.Cu) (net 1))
 (segment (start 39.624 32.512) (end 39.624 29.5656) (width 0.254) (layer F.Cu) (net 1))
 (segment (start 39.624 29.5656) (end 39.624 29.337) (width 0.254) (layer F.Cu) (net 1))
 (segment (start 47.9425 32.131) (end 50.6095 32.131) (width 0.254) (layer F.Cu) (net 13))
 (segment (start 50.6095 32.131) (end 50.8635 32.385) (width 0.254) (layer F.Cu) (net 13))
 (segment (start 33.4264 35.941) (end 33.4264 38.15588) (width 0.254) (layer F.Cu) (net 12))
 (segment (start 33.4264 38.15588) (end 33.3756 38.20668) (width 0.254) (layer F.Cu) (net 12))
 (segment (start 36.83 36.322) (end 34.8488 36.322) (width 0.254) (layer F.Cu) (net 12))
 (segment (start 34.4678 35.941) (end 33.4264 35.941) (width 0.254) (layer F.Cu) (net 12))
 (segment (start 34.8488 36.322) (end 34.4678 35.941) (width 0.254) (layer F.Cu) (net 12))
 (segment (start 46.101 36.322) (end 45.1485 36.322) (width 0.254) (layer F.Cu) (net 2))
 (segment (start 43.6245 33.782) (end 42.418 33.782) (width 0.254) (layer F.Cu) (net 2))
 (segment (start 43.688 33.8455) (end 43.6245 33.782) (width 0.254) (layer F.Cu) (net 2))
 (segment (start 43.688 34.8615) (end 43.688 33.8455) (width 0.254) (layer F.Cu) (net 2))
 (segment (start 45.1485 36.322) (end 43.688 34.8615) (width 0.254) (layer F.Cu) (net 2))
 (segment (start 48.8315 38.481) (end 46.7995 38.481) (width 0.254) (layer F.Cu) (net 2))
 (segment (start 46.101 37.7825) (end 46.101 36.322) (width 0.254) (layer F.Cu) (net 2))
 (segment (start 46.7995 38.481) (end 46.101 37.7825) (width 0.254) (layer F.Cu) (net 2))
 (segment (start 48.514 38.0365) (end 48.9585 38.481) (width 0.254) (layer F.Cu) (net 2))
 (segment (start 41.1607 26.1874) (end 41.1607 26.9113) (width 0.254) (layer F.Cu) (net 4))
 (segment (start 40.9956 31.242) (end 42.418 31.242) (width 0.254) (layer F.Cu) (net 4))
 (segment (start 40.64 30.8864) (end 40.9956 31.242) (width 0.254) (layer F.Cu) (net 4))
 (segment (start 40.64 27.432) (end 40.64 30.8864) (width 0.254) (layer F.Cu) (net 4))
 (segment (start 41.1607 26.9113) (end 40.64 27.432) (width 0.254) (layer F.Cu) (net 4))
 (segment (start 42.418 31.242) (end 43.815 31.242) (width 0.254) (layer F.Cu) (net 4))
 (segment (start 43.815 31.242) (end 44.831 32.258) (width 0.254) (layer F.Cu) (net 4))
 (segment (start 44.831 32.258) (end 45.9105 32.258) (width 0.254) (layer F.Cu) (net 4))
 (segment (start 45.9105 32.258) (end 46.0375 32.131) (width 0.254) (layer F.Cu) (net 4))
 (segment (start 41.1607 23.6474) (end 41.1607 26.1874) (width 0.254) (layer F.Cu) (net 4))
 (segment (start 42.799 22.2504) (end 42.799 21.463) (width 0.254) (layer F.Cu) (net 5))
 (segment (start 42.6974 21.3614) (end 41.1607 21.3614) (width 0.254) (layer F.Cu) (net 5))
 (segment (start 42.799 21.463) (end 42.6974 21.3614) (width 0.254) (layer F.Cu) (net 5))
 (segment (start 42.418 29.972) (end 41.275 29.972) (width 0.254) (layer F.Cu) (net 5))
 (segment (start 41.275 27.94) (end 43.053 26.162) (width 0.254) (layer F.Cu) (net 5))
 (segment (start 41.275 29.972) (end 41.275 27.94) (width 0.254) (layer F.Cu) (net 5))
 (segment (start 42.799 22.987) (end 42.799 25.908) (width 0.254) (layer F.Cu) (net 5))
 (segment (start 43.30192 26.28392) (end 45.085 26.28392) (width 0.254) (layer F.Cu) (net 5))
 (segment (start 43.17492 26.28392) (end 43.30192 26.28392) (width 0.254) (layer F.Cu) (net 5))
 (segment (start 42.799 25.908) (end 43.053 26.162) (width 0.254) (layer F.Cu) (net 5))
 (segment (start 43.053 26.162) (end 43.17492 26.28392) (width 0.254) (layer F.Cu) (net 5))
 (segment (start 46.2915 28.575) (end 46.2915 28.2575) (width 0.254) (layer F.Cu) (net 5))
 (segment (start 47.498 27.051) (end 47.498 26.28392) (width 0.254) (layer F.Cu) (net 5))
 (segment (start 46.2915 28.2575) (end 47.498 27.051) (width 0.254) (layer F.Cu) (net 5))
 (segment (start 42.799 23.114) (end 42.799 22.987) (width 0.254) (layer F.Cu) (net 5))
 (segment (start 42.799 22.987) (end 42.799 22.2504) (width 0.254) (layer F.Cu) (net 5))
 (segment (start 42.799 22.2504) (end 42.799 21.971) (width 0.254) (layer F.Cu) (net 5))
 (segment (start 42.799 22.733) (end 42.799 23.114) (width 0.254) (layer F.Cu) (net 5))
 (segment (start 44.831 26.28392) (end 47.498 26.28392) (width 0.254) (layer F.Cu) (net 5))
 (segment (start 47.498 26.28392) (end 49.657 26.28392) (width 0.254) (layer F.Cu) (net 5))
 (segment (start 44.831 26.28392) (end 44.831 27.1145) (width 0.254) (layer F.Cu) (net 5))
 (segment (start 44.831 27.1145) (end 46.2915 28.575) (width 0.254) (layer F.Cu) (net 5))
 (segment (start 44.20108 26.28392) (end 44.831 26.28392) (width 0.254) (layer F.Cu) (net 5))
 (segment (start 46.0629 19.939) (end 53.5432 19.939) (width 0.254) (layer F.Cu) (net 6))
 (segment (start 53.975 21.209) (end 53.975 27.686) (width 0.254) (layer F.Cu) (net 6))
 (segment (start 53.975 21.082) (end 53.975 21.209) (width 0.254) (layer F.Cu) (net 6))
 (segment (start 53.975 20.3708) (end 53.975 21.082) (width 0.254) (layer F.Cu) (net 6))
 (segment (start 53.5432 19.939) (end 53.975 20.3708) (width 0.254) (layer F.Cu) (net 6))
 (segment (start 52.7685 32.385) (end 52.7685 30.6705) (width 0.254) (layer F.Cu) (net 6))
 (segment (start 52.7685 30.6705) (end 52.6415 30.5435) (width 0.254) (layer F.Cu) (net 6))
 (segment (start 42.418 28.702) (end 44.2595 28.702) (width 0.254) (layer F.Cu) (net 6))
 (segment (start 44.2595 28.702) (end 44.3865 28.575) (width 0.254) (layer F.Cu) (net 6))
 (segment (start 48.3235 30.5435) (end 52.6415 30.5435) (width 0.254) (layer F.Cu) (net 6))
 (segment (start 52.6415 30.5435) (end 52.7685 30.5435) (width 0.254) (layer F.Cu) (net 6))
 (segment (start 52.7685 30.5435) (end 52.7685 28.8925) (width 0.254) (layer F.Cu) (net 6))
 (segment (start 52.7685 28.8925) (end 53.086 28.575) (width 0.254) (layer F.Cu) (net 6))
 (segment (start 53.086 28.575) (end 53.721 28.575) (width 0.254) (layer F.Cu) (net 6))
 (segment (start 53.975 28.321) (end 53.975 27.813) (width 0.254) (layer F.Cu) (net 6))
 (segment (start 53.721 28.575) (end 53.975 28.321) (width 0.254) (layer F.Cu) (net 6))
 (segment (start 44.3865 28.575) (end 44.3865 30.0355) (width 0.254) (layer F.Cu) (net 6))
 (segment (start 48.4505 30.4165) (end 48.4505 29.21) (width 0.254) (layer F.Cu) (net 6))
 (segment (start 48.133 30.734) (end 48.3235 30.5435) (width 0.254) (layer F.Cu) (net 6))
 (segment (start 48.3235 30.5435) (end 48.4505 30.4165) (width 0.254) (layer F.Cu) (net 6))
 (segment (start 45.085 30.734) (end 48.133 30.734) (width 0.254) (layer F.Cu) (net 6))
 (segment (start 44.3865 30.0355) (end 45.085 30.734) (width 0.254) (layer F.Cu) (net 6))
 (segment (start 44.1325 28.321) (end 44.3865 28.575) (width 0.254) (layer F.Cu) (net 6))
 (segment (start 40.0558 19.939) (end 40.0558 17.3282) (width 0.254) (layer F.Cu) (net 9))
 (segment (start 40.0558 17.3282) (end 39.8726 17.145) (width 0.254) (layer F.Cu) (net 9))
 (segment (start 35.5473 21.4376) (end 35.5473 20.1803) (width 0.254) (layer F.Cu) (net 9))
 (segment (start 35.7886 19.939) (end 40.0558 19.939) (width 0.254) (layer F.Cu) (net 9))
 (segment (start 40.0558 19.939) (end 44.1579 19.939) (width 0.254) (layer F.Cu) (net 9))
 (segment (start 35.5473 20.1803) (end 35.7886 19.939) (width 0.254) (layer F.Cu) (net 9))
 (segment (start 35.5473 21.4376) (end 33.909 21.4376) (width 0.254) (layer F.Cu) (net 9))
 (segment (start 36.5252 25.4508) (end 36.5252 22.6568) (width 0.254) (layer F.Cu) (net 9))
 (segment (start 35.5473 21.6789) (end 35.5473 21.4376) (width 0.254) (layer F.Cu) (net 9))
 (segment (start 36.5252 22.6568) (end 35.5473 21.6789) (width 0.254) (layer F.Cu) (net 9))
 (segment (start 36.83 31.242) (end 38.608 31.242) (width 0.254) (layer F.Cu) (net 9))
 (segment (start 36.5252 27.0256) (end 36.5252 25.4508) (width 0.254) (layer F.Cu) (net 9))
 (segment (start 36.5252 25.4508) (end 36.5252 25.0952) (width 0.254) (layer F.Cu) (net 9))
 (segment (start 36.7284 27.2288) (end 36.5252 27.0256) (width 0.254) (layer F.Cu) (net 9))
 (segment (start 38.1508 27.2288) (end 36.7284 27.2288) (width 0.254) (layer F.Cu) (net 9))
 (segment (start 38.6588 27.7368) (end 38.1508 27.2288) (width 0.254) (layer F.Cu) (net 9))
 (segment (start 38.6588 31.1912) (end 38.6588 27.7368) (width 0.254) (layer F.Cu) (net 9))
 (segment (start 38.608 31.242) (end 38.6588 31.1912) (width 0.254) (layer F.Cu) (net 9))
 (segment (start 43.1292 37.1348) (end 43.8023 37.1348) (width 0.254) (layer F.Cu) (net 10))
 (segment (start 41.1607 37.1348) (end 43.1292 37.1348) (width 0.254) (layer F.Cu) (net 10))
 (segment (start 42.8352 44.3122) (end 42.829 44.3122) (width 0.254) (layer F.Cu) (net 10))
 (segment (start 43.9674 43.18) (end 42.8352 44.3122) (width 0.254) (layer F.Cu) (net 10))
 (segment (start 43.9674 37.2999) (end 43.9674 43.18) (width 0.254) (layer F.Cu) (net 10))
 (segment (start 43.8023 37.1348) (end 43.9674 37.2999) (width 0.254) (layer F.Cu) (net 10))
 (segment (start 43.33206 45.620293) (end 43.080293 45.620293) (width 0.254) (layer F.Cu) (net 10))
 (segment (start 43.080293 45.620293) (end 42.829 45.369) (width 0.254) (layer F.Cu) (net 10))
 (segment (start 42.829 45.369) (end 42.829 44.3122) (width 0.254) (layer F.Cu) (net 10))
 (segment (start 43.18 45.593) (end 43.33206 45.620293) (width 0.254) (layer F.Cu) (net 10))
 (segment (start 43.33206 45.620293) (end 43.6753 45.6819) (width 0.254) (layer F.Cu) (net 10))
 (segment (start 43.6753 45.6819) (end 50.2158 45.6819) (width 0.254) (layer F.Cu) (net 10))
 (segment (start 50.2158 45.6819) (end 50.6135 45.589) (width 0.254) (layer F.Cu) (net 10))
 (segment (start 50.6135 45.589) (end 50.6135 44.3865) (width 0.254) (layer F.Cu) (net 10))
 (segment (start 50.8 36.3855) (end 48.5775 36.3855) (width 0.254) (layer F.Cu) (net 10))
 (segment (start 48.5775 36.3855) (end 48.514 36.322) (width 0.254) (layer F.Cu) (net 10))
 (segment (start 50.7365 38.481) (end 50.7365 36.449) (width 0.254) (layer F.Cu) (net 10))
 (segment (start 50.7365 36.449) (end 50.8 36.3855) (width 0.254) (layer F.Cu) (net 10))
 (segment (start 38.6715 32.512) (end 39.751 33.3375) (width 0.254) (layer F.Cu) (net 10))
 (segment (start 39.751 33.3375) (end 39.751 36.2585) (width 0.254) (layer F.Cu) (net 10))
 (segment (start 39.751 36.2585) (end 41.1607 37.1348) (width 0.254) (layer F.Cu) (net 10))
 (segment (start 41.1607 37.1348) (end 41.0972 37.0713) (width 0.254) (layer F.Cu) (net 10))
 (segment (start 36.83 32.512) (end 38.6715 32.512) (width 0.254) (layer F.Cu) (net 10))
 (segment (start 50.6135 44.3865) (end 50.6135 38.604) (width 0.254) (layer F.Cu) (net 10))
 (segment (start 50.6135 38.604) (end 50.7365 38.481) (width 0.254) (layer F.Cu) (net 10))
 (segment (start 38.9636 36.4617) (end 38.9636 36.6649) (width 0.254) (layer F.Cu) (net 7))
 (segment (start 37.7298 44.3122) (end 37.729 44.3122) (width 0.254) (layer F.Cu) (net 7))
 (segment (start 39.4589 42.5831) (end 37.7298 44.3122) (width 0.254) (layer F.Cu) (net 7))
 (segment (start 39.4589 37.1602) (end 39.4589 42.5831) (width 0.254) (layer F.Cu) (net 7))
 (segment (start 38.9636 36.6649) (end 39.4589 37.1602) (width 0.254) (layer F.Cu) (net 7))
 (segment (start 38.6334 33.782) (end 36.83 33.782) (width 0.254) (layer F.Cu) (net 7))
 (segment (start 38.9636 34.1122) (end 38.6334 33.782) (width 0.254) (layer F.Cu) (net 7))
 (segment (start 38.9636 36.5252) (end 38.9636 36.4617) (width 0.254) (layer F.Cu) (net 7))
 (segment (start 38.9636 36.4617) (end 38.9636 34.1122) (width 0.254) (layer F.Cu) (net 7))
 (segment (start 34.8615 32.004) (end 34.8615 33.4137) (width 0.254) (layer F.Cu) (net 7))
 (segment (start 35.2298 33.782) (end 36.83 33.782) (width 0.254) (layer F.Cu) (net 7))
 (segment (start 34.8615 33.4137) (end 35.2298 33.782) (width 0.254) (layer F.Cu) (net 7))
 (segment (start 36.83 28.702) (end 35.4584 28.702) (width 0.254) (layer F.Cu) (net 7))
 (segment (start 35.4584 28.702) (end 34.8615 29.2989) (width 0.254) (layer F.Cu) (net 7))
 (segment (start 34.8615 29.2989) (end 34.8615 32.004) (width 0.254) (layer F.Cu) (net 7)))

